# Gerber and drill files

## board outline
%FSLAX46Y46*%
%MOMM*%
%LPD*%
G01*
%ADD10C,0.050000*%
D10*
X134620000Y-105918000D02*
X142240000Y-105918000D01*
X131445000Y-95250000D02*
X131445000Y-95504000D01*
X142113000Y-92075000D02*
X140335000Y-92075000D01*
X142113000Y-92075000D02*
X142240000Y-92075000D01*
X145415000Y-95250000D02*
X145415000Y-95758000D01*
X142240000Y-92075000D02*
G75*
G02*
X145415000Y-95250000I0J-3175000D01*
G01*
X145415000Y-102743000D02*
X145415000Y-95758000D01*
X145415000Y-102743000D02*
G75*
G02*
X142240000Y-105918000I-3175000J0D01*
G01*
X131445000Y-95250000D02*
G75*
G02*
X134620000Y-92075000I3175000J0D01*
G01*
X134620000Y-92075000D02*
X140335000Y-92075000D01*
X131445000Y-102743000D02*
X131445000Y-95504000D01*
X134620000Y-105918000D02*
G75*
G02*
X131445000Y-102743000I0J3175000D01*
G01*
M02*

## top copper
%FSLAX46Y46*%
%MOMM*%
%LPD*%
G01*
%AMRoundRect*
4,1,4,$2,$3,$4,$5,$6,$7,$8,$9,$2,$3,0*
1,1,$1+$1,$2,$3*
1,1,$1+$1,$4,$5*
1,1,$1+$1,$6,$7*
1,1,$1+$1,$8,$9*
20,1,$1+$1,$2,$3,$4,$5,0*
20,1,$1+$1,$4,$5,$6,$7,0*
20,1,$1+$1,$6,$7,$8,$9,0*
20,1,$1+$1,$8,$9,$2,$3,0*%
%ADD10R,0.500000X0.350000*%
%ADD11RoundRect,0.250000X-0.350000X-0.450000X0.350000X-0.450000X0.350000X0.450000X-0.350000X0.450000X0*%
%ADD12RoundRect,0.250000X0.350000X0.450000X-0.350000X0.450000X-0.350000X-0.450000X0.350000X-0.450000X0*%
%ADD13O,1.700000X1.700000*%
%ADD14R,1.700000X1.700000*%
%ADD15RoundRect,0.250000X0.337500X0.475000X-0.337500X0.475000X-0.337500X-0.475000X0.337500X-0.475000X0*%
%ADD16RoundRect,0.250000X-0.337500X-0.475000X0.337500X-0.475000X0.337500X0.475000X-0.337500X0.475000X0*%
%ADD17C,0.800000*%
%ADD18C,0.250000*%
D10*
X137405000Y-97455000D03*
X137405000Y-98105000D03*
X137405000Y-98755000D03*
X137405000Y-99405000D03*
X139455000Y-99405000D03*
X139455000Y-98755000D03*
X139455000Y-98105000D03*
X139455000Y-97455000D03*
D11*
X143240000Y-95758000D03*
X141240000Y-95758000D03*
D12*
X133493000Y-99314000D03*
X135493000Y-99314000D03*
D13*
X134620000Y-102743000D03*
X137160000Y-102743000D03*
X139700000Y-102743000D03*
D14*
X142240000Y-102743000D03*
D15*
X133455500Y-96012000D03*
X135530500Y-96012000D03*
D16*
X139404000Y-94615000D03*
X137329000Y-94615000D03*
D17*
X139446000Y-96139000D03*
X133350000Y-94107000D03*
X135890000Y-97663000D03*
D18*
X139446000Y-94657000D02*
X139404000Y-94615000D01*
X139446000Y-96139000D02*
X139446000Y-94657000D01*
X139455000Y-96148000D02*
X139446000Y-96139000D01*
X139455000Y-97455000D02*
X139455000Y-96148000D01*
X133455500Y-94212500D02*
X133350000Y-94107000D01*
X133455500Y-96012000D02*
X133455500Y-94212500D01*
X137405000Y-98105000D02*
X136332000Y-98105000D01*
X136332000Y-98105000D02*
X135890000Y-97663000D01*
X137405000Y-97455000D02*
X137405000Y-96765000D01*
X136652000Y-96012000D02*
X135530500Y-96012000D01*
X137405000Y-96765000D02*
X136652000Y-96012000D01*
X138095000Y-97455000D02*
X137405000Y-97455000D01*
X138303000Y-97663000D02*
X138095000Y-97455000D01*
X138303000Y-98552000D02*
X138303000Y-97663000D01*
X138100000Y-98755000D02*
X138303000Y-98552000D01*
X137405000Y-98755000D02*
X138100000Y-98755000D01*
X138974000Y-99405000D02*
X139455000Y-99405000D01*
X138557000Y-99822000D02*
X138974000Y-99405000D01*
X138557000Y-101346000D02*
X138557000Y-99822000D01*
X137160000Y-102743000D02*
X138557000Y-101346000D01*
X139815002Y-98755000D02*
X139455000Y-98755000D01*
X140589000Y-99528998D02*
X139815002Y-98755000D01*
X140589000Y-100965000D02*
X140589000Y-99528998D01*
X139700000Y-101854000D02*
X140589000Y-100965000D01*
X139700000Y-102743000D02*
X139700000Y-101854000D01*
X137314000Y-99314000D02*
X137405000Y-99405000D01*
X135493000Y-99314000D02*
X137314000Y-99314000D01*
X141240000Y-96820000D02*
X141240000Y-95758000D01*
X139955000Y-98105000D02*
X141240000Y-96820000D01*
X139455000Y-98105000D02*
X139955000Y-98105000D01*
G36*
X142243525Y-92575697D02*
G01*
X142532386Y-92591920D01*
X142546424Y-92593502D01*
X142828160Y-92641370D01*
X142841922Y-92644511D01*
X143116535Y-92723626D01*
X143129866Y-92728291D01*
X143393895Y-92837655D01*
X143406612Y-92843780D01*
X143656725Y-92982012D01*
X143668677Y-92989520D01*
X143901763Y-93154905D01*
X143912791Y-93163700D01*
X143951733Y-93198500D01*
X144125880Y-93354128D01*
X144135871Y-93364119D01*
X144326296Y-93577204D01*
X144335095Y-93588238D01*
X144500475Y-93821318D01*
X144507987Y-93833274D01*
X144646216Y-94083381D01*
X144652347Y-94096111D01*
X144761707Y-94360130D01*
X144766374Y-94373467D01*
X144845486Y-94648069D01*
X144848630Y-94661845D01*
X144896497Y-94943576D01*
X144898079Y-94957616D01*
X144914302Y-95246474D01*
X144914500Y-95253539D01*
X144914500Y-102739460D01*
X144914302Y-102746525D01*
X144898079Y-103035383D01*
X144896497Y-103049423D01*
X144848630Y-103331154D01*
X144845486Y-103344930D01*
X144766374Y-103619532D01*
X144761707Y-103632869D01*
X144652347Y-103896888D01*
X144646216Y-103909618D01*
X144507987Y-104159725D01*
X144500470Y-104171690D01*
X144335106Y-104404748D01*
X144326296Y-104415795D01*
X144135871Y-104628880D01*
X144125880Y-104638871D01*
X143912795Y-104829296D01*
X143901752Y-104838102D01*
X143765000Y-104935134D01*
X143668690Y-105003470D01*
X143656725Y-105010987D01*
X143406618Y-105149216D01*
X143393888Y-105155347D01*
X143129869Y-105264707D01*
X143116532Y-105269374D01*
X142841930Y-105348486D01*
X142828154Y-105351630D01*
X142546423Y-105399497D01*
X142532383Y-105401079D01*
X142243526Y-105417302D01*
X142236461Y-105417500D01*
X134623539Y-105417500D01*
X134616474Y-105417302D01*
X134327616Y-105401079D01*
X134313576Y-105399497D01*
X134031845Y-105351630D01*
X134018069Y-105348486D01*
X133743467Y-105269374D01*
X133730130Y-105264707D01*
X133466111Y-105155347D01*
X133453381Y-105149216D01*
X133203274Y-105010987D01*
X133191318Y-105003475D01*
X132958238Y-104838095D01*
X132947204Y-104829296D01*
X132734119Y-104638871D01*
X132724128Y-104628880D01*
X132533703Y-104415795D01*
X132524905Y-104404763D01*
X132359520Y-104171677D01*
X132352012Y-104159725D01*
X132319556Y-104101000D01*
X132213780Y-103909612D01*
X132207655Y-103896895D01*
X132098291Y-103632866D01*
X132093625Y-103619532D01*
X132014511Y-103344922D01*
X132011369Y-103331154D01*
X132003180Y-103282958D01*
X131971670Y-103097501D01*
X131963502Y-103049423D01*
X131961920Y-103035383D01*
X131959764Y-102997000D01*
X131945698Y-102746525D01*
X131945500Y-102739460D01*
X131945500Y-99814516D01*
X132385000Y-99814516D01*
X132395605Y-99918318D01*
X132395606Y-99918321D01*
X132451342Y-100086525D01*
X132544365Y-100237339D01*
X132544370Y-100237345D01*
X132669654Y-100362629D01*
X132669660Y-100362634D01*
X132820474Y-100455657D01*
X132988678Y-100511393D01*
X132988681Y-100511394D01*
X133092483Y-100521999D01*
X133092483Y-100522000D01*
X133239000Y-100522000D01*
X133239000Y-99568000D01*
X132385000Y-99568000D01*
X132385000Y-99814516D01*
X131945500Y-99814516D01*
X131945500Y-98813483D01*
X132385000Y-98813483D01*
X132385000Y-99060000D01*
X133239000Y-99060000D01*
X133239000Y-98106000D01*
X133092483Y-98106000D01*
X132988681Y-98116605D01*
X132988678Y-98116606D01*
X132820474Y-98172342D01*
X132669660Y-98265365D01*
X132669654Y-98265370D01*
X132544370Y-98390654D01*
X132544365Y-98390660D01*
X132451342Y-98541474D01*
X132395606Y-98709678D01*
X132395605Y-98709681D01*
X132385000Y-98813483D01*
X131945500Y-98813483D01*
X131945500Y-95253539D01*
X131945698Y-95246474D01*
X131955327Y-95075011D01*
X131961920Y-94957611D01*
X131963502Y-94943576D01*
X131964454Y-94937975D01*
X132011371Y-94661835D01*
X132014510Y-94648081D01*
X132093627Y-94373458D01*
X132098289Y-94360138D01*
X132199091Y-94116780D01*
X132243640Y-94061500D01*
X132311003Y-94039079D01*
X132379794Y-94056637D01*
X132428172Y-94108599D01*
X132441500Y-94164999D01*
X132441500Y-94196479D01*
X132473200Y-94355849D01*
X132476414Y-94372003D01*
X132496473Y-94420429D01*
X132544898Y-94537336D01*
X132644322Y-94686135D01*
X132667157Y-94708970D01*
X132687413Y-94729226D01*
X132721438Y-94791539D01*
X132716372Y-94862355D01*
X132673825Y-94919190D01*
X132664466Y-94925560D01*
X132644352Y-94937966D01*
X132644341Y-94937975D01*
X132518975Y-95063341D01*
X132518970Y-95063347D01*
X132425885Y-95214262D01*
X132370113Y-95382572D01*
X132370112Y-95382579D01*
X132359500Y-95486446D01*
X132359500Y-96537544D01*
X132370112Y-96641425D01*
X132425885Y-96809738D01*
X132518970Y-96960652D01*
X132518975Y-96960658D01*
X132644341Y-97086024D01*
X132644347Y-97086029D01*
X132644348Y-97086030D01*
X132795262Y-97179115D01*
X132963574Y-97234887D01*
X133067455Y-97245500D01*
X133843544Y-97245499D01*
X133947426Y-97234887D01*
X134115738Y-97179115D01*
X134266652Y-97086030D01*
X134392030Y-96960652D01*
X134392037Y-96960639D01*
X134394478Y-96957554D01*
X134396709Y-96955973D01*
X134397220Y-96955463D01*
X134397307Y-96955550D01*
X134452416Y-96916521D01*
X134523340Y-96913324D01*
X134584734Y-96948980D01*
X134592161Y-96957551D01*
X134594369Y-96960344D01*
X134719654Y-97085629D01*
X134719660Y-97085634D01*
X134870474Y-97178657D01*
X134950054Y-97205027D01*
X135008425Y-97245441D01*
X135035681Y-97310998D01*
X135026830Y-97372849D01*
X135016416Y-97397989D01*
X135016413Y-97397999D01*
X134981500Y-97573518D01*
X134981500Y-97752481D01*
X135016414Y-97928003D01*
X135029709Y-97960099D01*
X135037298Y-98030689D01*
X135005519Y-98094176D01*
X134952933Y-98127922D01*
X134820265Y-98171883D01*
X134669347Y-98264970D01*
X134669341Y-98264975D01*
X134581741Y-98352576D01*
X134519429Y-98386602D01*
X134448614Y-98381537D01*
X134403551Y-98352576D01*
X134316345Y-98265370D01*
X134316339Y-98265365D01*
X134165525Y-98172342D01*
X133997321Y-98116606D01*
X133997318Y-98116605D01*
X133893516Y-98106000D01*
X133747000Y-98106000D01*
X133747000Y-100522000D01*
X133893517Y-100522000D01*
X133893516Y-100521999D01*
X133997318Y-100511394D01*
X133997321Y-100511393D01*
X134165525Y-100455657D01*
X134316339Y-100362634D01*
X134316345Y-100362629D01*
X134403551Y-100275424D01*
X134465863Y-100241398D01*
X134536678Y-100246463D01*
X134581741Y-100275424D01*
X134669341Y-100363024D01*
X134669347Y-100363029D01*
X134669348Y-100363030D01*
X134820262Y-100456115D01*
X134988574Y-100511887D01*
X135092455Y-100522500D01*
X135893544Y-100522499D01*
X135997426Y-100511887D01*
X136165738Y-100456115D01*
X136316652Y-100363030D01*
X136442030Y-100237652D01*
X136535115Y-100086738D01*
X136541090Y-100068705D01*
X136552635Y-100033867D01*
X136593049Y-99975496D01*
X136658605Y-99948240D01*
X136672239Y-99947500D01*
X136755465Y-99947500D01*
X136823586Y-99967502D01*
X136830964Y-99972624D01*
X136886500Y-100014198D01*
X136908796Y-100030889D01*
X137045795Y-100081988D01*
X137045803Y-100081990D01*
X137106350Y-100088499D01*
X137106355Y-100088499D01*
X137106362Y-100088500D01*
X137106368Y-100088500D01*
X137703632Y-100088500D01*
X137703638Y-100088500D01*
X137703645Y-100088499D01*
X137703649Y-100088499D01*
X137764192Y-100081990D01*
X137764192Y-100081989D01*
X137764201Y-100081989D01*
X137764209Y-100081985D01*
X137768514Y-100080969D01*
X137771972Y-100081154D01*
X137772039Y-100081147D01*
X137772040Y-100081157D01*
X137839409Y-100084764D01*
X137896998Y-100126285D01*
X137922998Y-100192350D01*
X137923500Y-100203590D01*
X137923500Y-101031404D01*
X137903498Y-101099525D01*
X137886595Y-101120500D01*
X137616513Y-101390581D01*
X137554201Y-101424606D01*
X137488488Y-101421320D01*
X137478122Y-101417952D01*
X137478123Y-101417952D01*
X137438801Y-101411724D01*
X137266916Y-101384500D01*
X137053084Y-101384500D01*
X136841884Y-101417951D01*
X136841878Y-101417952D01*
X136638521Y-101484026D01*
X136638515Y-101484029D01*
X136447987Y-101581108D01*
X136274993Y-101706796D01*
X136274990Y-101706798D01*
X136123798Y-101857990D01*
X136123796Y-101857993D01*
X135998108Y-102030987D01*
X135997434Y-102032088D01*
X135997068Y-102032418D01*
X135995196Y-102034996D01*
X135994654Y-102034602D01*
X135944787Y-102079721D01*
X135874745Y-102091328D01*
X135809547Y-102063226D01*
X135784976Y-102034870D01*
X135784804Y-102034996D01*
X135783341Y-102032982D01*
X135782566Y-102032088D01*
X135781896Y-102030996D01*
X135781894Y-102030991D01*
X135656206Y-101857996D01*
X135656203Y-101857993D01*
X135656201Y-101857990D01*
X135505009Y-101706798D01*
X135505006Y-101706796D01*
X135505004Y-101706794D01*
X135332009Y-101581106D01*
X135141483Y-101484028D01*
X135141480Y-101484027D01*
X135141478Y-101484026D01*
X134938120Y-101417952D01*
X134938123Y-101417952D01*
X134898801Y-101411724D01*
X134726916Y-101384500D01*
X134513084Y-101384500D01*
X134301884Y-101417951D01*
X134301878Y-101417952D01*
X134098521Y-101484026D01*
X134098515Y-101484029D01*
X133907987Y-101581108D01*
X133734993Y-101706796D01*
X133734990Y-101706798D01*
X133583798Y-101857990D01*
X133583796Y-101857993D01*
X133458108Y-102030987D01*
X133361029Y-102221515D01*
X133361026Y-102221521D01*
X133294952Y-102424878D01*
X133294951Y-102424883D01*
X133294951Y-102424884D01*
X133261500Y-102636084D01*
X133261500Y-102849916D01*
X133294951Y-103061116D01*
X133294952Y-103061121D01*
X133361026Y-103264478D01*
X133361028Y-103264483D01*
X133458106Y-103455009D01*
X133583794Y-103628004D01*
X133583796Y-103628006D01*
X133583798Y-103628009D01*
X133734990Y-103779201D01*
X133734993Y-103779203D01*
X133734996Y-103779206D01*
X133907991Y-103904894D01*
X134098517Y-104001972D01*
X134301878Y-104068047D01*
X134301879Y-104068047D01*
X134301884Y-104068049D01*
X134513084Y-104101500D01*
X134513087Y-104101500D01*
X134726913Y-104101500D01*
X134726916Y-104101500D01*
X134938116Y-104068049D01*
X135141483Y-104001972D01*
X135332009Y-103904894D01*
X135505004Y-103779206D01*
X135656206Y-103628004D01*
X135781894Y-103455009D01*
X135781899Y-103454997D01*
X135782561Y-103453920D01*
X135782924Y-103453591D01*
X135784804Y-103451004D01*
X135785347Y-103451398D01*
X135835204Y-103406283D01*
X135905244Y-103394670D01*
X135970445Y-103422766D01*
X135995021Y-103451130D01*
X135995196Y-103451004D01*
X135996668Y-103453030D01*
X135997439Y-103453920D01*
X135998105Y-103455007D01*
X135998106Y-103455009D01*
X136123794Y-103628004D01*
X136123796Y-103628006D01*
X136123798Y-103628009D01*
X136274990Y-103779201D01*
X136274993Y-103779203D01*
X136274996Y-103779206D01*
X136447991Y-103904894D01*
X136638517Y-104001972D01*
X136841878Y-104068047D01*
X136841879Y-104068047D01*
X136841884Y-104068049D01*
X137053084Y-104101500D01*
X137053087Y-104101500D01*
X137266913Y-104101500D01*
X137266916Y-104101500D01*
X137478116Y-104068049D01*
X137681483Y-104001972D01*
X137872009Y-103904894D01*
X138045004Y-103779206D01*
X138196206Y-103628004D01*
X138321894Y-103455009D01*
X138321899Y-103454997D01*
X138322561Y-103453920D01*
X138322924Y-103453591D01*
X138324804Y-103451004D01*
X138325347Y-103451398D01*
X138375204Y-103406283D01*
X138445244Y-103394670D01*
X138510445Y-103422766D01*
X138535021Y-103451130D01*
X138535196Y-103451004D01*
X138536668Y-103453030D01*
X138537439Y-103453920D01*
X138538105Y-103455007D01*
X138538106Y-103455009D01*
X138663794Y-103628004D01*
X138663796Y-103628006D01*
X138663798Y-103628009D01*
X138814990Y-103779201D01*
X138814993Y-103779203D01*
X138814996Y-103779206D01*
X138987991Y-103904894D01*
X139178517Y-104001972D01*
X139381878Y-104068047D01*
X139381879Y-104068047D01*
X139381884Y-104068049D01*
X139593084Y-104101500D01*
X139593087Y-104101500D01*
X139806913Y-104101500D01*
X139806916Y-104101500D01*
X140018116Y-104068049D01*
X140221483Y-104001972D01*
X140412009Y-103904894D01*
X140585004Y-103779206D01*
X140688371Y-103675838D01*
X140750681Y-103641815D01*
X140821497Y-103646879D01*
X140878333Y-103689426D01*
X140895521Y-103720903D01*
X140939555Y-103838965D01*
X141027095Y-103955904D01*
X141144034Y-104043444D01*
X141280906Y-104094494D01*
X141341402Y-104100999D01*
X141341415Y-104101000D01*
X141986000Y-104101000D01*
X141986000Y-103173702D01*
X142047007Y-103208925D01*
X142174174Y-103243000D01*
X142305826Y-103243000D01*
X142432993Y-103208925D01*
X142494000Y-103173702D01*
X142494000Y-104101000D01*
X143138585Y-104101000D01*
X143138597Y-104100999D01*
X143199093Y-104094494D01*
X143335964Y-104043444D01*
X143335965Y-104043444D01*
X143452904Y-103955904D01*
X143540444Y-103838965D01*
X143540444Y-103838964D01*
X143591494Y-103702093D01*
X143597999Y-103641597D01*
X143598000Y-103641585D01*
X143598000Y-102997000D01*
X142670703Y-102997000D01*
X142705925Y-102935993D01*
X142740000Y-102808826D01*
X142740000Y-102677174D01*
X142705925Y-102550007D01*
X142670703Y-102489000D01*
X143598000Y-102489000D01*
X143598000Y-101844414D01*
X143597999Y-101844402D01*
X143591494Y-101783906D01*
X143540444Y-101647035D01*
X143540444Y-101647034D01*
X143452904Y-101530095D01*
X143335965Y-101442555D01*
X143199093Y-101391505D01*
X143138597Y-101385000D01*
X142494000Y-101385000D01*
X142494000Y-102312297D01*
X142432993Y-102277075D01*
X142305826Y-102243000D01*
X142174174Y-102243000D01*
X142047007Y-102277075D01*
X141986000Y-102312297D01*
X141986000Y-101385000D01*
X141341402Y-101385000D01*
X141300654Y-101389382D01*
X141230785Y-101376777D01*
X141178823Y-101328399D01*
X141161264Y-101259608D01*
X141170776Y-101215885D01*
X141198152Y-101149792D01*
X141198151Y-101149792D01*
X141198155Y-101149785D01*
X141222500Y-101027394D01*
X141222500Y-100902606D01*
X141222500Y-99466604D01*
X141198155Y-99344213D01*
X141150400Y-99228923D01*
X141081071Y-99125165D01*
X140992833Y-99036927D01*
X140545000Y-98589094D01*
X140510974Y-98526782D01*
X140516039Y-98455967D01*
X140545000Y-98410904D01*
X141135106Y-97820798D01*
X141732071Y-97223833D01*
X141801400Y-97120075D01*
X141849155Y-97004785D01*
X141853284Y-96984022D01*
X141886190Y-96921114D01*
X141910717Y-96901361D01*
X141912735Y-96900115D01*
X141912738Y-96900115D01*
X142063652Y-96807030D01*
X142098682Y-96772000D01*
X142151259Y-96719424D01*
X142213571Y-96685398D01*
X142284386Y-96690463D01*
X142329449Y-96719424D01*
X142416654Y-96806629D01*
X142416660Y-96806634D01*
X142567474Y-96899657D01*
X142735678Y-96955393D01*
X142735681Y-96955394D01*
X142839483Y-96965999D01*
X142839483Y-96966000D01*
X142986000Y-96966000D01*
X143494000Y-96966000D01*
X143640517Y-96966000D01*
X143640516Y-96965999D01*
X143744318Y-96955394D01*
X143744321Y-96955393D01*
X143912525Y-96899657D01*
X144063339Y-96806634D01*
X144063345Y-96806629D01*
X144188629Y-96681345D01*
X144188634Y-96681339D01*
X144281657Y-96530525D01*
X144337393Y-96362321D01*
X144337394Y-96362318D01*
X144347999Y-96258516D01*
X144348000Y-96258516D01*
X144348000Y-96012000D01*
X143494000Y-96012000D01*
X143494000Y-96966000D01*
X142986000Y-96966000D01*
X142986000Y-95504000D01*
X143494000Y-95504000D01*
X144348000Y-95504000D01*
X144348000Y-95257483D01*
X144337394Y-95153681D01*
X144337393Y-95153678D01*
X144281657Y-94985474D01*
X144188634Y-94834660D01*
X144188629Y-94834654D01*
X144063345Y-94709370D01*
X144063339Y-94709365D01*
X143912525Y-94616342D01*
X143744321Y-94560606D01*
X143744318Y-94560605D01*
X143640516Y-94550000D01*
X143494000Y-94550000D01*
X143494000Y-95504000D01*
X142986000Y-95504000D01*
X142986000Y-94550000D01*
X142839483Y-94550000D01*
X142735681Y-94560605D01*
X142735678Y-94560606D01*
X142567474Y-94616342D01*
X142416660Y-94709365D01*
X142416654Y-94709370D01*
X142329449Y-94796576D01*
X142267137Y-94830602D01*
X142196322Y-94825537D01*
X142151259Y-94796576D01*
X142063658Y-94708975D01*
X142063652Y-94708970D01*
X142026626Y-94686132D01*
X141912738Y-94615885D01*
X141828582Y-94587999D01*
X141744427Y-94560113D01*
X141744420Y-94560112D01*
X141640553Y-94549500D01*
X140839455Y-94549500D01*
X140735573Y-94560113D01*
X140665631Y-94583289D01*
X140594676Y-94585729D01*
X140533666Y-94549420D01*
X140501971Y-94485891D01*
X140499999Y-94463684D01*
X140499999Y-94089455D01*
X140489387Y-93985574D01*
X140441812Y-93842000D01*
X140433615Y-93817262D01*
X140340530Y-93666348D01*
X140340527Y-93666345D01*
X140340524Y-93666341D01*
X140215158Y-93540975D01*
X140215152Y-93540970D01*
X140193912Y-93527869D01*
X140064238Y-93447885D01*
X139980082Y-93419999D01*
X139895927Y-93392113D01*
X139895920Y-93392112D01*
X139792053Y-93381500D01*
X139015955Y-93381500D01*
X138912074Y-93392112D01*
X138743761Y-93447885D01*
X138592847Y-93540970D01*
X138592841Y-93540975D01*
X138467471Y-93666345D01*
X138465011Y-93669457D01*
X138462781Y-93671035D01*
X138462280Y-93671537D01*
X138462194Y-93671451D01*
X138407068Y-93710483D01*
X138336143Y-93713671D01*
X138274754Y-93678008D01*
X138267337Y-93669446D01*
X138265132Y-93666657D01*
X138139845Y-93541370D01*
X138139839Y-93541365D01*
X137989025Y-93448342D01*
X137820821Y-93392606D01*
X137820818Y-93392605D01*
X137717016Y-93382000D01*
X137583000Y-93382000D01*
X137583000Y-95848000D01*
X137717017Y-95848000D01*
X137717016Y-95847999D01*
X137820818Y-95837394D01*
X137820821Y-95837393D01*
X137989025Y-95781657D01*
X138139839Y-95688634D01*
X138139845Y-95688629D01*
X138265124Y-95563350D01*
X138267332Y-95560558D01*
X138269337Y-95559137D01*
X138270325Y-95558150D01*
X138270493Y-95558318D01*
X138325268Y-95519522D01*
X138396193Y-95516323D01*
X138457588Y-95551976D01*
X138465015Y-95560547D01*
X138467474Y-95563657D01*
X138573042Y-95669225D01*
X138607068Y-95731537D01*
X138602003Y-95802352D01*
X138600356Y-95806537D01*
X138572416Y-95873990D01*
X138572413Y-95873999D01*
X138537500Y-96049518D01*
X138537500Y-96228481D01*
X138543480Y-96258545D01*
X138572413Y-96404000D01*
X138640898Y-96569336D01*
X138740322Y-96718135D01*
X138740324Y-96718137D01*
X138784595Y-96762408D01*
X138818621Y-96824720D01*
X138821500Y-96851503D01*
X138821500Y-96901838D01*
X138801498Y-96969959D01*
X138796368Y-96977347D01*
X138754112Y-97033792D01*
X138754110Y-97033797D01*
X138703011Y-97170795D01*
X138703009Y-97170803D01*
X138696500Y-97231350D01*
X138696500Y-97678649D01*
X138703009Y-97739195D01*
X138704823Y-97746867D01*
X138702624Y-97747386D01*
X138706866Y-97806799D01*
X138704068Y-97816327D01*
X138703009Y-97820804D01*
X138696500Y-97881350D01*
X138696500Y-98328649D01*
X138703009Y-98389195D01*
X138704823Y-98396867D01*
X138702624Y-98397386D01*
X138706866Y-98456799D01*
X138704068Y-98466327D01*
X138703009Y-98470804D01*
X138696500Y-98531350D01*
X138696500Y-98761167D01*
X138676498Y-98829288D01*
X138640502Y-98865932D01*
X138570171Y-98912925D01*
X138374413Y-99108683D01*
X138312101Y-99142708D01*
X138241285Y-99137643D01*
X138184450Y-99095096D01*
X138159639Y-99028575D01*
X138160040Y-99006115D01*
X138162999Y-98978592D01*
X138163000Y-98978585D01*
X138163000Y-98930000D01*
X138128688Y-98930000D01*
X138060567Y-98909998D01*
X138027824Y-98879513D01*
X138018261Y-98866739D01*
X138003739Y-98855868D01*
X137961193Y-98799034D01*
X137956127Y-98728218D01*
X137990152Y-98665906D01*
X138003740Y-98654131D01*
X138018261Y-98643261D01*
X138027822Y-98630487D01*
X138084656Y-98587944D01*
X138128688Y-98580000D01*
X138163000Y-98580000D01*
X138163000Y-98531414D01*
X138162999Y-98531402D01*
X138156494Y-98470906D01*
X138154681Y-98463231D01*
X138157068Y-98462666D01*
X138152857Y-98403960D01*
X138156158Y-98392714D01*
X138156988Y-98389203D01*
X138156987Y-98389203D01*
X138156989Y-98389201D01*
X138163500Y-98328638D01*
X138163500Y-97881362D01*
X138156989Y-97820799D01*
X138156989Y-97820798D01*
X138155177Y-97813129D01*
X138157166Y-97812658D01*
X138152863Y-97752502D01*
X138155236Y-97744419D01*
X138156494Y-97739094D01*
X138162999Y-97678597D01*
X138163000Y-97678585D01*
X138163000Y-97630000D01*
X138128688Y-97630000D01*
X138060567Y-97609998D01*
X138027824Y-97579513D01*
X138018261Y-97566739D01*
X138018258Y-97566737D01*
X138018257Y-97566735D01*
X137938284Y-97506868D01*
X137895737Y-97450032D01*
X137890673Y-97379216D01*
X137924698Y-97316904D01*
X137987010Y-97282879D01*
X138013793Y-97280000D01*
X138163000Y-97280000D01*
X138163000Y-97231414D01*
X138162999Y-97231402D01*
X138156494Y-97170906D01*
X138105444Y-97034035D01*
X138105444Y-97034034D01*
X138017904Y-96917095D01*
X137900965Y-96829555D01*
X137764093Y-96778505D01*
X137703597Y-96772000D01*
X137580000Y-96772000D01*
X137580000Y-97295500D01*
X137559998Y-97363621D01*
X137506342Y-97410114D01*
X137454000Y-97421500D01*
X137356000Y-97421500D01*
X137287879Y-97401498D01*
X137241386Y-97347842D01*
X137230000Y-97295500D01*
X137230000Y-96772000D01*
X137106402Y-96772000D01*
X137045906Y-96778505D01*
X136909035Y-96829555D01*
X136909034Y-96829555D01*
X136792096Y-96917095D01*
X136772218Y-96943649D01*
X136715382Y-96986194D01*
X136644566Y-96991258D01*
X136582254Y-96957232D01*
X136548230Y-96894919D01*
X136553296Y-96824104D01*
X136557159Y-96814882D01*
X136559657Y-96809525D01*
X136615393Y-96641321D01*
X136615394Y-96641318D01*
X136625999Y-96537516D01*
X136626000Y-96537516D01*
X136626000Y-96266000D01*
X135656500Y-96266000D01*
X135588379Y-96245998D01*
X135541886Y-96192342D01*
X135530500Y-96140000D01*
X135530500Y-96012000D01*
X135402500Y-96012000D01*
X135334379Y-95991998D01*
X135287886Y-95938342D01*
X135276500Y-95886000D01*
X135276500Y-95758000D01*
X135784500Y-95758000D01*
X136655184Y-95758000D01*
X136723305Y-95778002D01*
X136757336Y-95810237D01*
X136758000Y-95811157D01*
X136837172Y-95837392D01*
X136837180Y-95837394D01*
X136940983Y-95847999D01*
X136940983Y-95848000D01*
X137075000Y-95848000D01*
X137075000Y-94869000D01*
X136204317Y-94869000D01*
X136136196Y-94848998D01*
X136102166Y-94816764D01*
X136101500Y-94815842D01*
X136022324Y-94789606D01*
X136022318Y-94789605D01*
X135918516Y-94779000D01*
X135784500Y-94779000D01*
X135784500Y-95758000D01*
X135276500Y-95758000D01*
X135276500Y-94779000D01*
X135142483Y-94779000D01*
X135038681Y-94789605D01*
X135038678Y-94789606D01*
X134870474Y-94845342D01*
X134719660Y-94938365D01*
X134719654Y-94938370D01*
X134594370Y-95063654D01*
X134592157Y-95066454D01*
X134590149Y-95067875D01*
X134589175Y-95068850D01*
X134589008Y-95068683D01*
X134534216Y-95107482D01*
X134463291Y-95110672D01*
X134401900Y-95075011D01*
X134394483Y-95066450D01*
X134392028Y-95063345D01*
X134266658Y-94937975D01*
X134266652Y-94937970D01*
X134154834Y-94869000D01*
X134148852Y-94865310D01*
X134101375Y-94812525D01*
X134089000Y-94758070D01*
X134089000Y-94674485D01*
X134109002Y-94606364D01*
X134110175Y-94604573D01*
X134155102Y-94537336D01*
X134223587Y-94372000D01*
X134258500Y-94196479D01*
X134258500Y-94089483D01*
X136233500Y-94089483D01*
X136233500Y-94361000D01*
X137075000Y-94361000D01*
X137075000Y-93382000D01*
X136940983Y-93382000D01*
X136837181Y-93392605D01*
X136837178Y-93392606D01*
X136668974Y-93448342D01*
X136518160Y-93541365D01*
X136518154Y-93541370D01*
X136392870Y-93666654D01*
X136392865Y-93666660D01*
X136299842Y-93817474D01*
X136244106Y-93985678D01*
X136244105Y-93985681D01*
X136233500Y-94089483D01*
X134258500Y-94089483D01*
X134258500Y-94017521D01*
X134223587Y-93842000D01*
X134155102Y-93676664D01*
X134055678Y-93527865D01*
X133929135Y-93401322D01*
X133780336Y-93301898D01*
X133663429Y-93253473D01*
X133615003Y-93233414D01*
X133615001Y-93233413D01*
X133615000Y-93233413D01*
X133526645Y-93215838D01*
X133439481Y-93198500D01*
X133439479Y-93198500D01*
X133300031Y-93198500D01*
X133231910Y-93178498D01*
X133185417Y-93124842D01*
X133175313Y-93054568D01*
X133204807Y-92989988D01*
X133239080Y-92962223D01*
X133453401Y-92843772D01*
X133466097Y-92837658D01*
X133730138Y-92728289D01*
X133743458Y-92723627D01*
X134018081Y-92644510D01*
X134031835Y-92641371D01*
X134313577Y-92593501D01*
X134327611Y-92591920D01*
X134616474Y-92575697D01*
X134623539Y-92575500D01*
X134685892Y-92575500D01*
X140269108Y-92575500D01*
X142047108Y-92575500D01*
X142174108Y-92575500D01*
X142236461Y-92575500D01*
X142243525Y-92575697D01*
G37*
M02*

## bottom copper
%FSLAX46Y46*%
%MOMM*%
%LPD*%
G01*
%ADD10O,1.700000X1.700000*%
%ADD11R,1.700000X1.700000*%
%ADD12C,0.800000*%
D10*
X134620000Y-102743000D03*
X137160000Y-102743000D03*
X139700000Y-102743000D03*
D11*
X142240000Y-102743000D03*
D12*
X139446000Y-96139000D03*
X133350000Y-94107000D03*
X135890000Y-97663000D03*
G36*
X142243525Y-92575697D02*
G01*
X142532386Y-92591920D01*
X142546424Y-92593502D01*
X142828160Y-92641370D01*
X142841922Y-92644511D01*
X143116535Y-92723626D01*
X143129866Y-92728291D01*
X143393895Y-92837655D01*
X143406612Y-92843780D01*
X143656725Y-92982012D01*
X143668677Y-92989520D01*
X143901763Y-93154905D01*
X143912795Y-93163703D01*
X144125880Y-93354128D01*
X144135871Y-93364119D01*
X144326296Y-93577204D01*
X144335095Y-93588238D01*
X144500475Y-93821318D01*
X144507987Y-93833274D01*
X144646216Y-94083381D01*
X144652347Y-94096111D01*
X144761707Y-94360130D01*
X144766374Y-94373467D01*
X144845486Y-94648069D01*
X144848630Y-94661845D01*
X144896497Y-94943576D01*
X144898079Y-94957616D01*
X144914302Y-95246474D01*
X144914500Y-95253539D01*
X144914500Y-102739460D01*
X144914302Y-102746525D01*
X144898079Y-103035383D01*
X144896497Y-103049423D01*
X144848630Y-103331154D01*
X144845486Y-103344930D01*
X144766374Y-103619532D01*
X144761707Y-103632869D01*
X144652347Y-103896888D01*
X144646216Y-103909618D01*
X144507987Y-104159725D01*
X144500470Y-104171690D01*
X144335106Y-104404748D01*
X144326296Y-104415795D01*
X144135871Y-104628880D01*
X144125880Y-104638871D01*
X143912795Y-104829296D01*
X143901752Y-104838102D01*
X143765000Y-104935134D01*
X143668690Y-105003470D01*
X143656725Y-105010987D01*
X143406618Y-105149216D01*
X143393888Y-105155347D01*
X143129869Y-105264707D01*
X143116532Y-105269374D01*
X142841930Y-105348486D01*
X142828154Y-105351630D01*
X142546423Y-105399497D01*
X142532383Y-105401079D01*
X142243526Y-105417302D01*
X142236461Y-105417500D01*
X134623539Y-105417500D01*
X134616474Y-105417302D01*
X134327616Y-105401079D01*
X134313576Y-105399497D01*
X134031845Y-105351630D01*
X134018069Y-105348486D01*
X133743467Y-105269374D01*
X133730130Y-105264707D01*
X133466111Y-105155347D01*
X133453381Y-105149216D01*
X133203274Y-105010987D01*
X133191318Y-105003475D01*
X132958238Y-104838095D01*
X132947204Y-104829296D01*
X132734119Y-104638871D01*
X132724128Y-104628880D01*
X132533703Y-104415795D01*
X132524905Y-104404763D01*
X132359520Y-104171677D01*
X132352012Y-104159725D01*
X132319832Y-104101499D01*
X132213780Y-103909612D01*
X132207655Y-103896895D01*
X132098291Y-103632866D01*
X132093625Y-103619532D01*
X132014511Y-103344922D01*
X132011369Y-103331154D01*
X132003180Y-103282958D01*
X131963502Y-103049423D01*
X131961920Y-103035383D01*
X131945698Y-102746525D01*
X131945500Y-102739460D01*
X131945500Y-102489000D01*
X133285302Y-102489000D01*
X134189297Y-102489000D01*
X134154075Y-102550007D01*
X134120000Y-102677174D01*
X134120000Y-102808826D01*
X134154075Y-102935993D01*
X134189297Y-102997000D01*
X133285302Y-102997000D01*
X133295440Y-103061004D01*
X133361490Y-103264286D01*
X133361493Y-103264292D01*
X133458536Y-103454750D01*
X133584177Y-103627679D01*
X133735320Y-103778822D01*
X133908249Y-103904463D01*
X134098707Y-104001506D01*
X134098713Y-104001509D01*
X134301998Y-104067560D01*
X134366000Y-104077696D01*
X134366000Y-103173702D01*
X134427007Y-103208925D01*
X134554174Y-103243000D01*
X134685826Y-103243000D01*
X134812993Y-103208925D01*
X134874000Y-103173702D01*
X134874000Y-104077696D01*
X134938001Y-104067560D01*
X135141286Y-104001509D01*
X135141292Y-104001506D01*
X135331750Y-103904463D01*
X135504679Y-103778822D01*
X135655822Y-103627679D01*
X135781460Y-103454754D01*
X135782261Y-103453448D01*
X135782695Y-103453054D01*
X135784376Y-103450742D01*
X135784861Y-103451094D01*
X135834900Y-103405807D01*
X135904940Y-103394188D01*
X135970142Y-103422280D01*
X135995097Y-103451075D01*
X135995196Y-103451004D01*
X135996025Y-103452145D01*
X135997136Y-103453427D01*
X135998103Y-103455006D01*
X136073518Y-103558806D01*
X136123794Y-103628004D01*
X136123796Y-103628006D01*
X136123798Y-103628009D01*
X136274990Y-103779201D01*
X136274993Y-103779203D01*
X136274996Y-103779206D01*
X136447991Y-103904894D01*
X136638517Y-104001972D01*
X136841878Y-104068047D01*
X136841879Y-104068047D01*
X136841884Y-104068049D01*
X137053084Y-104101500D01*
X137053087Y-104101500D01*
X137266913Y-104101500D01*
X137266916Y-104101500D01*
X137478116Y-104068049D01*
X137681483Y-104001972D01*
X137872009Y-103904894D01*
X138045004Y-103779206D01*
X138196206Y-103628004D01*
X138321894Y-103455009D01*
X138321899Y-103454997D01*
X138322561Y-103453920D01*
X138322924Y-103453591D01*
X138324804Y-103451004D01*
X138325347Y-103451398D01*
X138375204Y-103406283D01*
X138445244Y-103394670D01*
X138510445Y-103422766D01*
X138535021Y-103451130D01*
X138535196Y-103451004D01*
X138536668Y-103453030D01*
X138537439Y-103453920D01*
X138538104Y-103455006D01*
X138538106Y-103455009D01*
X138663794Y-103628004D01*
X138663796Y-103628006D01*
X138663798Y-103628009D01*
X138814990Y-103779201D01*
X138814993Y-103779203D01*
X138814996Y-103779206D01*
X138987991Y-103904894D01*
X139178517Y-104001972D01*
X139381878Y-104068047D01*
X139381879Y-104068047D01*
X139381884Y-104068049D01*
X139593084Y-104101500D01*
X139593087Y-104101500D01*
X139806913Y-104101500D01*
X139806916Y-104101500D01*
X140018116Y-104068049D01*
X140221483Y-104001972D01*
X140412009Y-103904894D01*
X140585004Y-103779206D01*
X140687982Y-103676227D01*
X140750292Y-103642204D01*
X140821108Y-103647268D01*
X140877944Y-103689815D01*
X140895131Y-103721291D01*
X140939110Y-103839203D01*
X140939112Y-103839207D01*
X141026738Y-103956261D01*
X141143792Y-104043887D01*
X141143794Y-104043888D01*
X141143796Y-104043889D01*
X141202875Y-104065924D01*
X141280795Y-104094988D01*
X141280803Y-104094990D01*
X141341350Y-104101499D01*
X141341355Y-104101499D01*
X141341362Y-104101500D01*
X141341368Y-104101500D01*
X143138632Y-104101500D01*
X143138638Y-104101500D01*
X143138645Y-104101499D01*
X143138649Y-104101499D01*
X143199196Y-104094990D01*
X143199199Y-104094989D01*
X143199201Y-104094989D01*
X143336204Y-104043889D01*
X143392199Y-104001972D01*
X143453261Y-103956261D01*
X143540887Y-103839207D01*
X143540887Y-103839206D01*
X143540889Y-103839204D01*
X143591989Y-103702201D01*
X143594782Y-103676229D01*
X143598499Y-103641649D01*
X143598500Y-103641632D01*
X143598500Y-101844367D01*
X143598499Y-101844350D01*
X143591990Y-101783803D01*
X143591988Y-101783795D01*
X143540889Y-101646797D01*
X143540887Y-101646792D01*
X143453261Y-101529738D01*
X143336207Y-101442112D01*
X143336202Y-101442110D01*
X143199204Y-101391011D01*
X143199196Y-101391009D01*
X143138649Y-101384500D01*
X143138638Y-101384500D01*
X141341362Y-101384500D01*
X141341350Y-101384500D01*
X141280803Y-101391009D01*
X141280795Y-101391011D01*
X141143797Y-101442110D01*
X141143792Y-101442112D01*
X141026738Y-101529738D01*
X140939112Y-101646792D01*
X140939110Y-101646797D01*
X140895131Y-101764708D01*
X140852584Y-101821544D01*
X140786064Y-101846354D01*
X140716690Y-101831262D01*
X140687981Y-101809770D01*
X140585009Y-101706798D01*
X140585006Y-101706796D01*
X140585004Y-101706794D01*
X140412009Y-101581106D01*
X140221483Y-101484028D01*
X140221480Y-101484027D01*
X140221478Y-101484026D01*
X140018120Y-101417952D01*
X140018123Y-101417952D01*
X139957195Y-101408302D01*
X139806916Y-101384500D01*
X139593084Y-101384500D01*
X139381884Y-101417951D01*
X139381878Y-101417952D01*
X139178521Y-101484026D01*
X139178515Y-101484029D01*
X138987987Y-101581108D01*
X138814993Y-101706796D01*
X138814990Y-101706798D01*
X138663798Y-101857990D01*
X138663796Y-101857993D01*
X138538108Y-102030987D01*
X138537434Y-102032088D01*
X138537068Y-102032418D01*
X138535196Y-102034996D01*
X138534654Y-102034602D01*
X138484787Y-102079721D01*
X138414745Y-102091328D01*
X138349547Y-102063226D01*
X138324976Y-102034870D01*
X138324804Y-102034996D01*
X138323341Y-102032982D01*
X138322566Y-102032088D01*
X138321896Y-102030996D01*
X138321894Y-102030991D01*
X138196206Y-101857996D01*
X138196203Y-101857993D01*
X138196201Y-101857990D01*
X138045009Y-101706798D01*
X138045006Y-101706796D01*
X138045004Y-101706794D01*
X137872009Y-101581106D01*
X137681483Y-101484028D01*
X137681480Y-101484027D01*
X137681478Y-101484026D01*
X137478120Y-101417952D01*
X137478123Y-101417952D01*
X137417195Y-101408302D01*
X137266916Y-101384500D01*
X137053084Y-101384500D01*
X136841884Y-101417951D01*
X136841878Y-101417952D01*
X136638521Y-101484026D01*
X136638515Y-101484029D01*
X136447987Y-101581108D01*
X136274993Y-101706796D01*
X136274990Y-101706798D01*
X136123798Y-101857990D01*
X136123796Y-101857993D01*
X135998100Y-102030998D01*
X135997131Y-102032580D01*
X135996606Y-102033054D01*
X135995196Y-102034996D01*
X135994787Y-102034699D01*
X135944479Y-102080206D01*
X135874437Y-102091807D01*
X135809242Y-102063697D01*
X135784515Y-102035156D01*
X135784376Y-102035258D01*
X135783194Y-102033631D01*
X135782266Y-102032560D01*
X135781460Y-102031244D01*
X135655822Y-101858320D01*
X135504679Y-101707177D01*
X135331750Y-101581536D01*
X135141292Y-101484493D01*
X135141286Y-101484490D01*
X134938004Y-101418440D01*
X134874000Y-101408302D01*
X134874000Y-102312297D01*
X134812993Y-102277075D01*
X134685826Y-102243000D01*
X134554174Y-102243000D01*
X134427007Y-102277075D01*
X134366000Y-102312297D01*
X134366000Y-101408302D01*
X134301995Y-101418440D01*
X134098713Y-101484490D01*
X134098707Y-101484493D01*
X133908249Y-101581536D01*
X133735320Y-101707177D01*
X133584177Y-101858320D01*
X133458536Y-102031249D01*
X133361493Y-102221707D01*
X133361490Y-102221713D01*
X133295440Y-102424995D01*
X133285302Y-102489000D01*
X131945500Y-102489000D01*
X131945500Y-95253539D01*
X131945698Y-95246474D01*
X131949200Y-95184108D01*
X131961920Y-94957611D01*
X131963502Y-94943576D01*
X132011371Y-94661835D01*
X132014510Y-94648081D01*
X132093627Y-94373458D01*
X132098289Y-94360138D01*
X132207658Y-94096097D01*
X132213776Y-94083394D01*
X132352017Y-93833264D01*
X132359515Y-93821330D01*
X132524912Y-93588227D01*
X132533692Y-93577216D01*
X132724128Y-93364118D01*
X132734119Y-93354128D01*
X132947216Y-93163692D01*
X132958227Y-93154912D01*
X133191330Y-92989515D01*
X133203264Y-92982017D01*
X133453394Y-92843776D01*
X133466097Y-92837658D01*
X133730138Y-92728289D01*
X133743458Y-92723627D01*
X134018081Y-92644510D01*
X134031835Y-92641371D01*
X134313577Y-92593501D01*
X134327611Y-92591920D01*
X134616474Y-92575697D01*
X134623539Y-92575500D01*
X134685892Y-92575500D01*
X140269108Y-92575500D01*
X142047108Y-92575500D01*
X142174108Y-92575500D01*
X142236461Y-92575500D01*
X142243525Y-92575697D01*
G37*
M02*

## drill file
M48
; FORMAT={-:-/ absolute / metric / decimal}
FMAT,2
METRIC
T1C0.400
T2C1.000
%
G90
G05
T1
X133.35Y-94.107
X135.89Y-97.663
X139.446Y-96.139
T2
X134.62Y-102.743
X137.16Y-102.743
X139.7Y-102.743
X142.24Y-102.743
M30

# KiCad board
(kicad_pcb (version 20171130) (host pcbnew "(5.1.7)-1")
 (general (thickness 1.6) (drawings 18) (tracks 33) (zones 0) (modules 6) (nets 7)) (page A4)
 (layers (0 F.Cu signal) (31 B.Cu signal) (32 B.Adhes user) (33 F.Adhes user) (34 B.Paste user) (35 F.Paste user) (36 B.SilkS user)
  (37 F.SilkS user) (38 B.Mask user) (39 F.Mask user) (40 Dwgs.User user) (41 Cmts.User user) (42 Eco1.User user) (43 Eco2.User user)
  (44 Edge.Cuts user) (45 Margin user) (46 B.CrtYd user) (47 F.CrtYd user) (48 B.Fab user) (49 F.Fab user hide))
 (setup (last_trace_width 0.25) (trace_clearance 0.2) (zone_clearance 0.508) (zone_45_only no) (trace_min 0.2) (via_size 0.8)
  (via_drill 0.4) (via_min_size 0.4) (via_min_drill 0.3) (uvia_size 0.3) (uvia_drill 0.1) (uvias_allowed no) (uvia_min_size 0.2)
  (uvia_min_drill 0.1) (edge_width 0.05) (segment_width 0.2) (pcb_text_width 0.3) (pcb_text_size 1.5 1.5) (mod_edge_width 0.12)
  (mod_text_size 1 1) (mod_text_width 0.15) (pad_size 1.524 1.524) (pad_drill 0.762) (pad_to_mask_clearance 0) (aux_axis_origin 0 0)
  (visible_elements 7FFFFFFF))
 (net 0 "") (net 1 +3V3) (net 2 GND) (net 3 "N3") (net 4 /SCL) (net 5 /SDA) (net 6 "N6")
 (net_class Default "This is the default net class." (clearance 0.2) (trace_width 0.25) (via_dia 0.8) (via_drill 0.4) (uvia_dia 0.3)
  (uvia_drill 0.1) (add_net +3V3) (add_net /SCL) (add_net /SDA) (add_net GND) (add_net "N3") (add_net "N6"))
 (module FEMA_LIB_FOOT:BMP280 (layer F.Cu) (at 138.43 98.425)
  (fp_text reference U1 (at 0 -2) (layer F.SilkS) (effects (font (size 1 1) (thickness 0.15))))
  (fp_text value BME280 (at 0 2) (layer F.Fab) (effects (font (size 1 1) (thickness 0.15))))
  (pad 8 smd rect (at -1.025 -0.97) (size 0.5 0.35) (layers F.Cu F.Paste F.Mask) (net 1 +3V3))
  (pad 7 smd rect (at -1.025 -0.32) (size 0.5 0.35) (layers F.Cu F.Paste F.Mask) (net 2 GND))
  (pad 6 smd rect (at -1.025 0.33) (size 0.5 0.35) (layers F.Cu F.Paste F.Mask) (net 1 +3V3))
  (pad 5 smd rect (at -1.025 0.98) (size 0.5 0.35) (layers F.Cu F.Paste F.Mask) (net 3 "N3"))
  (pad 4 smd rect (at 1.025 0.98) (size 0.5 0.35) (layers F.Cu F.Paste F.Mask) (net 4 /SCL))
  (pad 3 smd rect (at 1.025 0.33) (size 0.5 0.35) (layers F.Cu F.Paste F.Mask) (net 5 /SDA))
  (pad 2 smd rect (at 1.025 -0.32) (size 0.5 0.35) (layers F.Cu F.Paste F.Mask) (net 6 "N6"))
  (pad 1 smd rect (at 1.025 -0.97) (size 0.5 0.35) (layers F.Cu F.Paste F.Mask) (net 2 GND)))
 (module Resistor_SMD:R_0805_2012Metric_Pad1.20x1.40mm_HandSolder (layer F.Cu) (at 142.24 95.758)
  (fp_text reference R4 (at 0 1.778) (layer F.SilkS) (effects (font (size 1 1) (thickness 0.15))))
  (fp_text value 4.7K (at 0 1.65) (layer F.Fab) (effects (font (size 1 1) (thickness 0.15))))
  (pad 2 smd roundrect (at 1 0) (size 1.2 1.4) (layers F.Cu F.Paste F.Mask) (roundrect_rratio 0.208333) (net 1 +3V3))
  (pad 1 smd roundrect (at -1 0) (size 1.2 1.4) (layers F.Cu F.Paste F.Mask) (roundrect_rratio 0.208333) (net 6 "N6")))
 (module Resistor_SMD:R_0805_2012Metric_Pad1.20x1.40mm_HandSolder (layer F.Cu) (at 134.493 99.314 180)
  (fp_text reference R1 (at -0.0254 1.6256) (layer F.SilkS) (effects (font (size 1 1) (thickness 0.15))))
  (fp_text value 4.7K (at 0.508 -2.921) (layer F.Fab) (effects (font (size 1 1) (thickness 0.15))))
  (pad 2 smd roundrect (at 1 0 180) (size 1.2 1.4) (layers F.Cu F.Paste F.Mask) (roundrect_rratio 0.208333) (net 1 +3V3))
  (pad 1 smd roundrect (at -1 0 180) (size 1.2 1.4) (layers F.Cu F.Paste F.Mask) (roundrect_rratio 0.208333) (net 3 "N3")))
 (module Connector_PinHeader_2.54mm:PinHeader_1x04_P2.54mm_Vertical (layer F.Cu) (at 142.24 102.743 270)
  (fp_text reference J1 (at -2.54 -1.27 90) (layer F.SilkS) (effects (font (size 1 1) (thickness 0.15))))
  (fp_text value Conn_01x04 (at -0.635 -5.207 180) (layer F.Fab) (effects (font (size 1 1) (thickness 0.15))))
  (pad 4 thru_hole oval (at 0 7.62 270) (size 1.7 1.7) (drill 1) (layers *.Cu *.Mask) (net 2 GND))
  (pad 3 thru_hole oval (at 0 5.08 270) (size 1.7 1.7) (drill 1) (layers *.Cu *.Mask) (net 4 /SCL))
  (pad 2 thru_hole oval (at 0 2.54 270) (size 1.7 1.7) (drill 1) (layers *.Cu *.Mask) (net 5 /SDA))
  (pad 1 thru_hole rect (at 0 0 270) (size 1.7 1.7) (drill 1) (layers *.Cu *.Mask) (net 1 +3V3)))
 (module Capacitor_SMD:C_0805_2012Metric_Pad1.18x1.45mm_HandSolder (layer F.Cu) (at 134.493 96.012 180)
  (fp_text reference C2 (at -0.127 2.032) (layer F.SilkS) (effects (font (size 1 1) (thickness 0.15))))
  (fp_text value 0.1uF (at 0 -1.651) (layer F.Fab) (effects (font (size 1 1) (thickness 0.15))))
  (pad 2 smd roundrect (at 1.0375 0 180) (size 1.175 1.45) (layers F.Cu F.Paste F.Mask) (roundrect_rratio 0.212766) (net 2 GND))
  (pad 1 smd roundrect (at -1.0375 0 180) (size 1.175 1.45) (layers F.Cu F.Paste F.Mask) (roundrect_rratio 0.212766) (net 1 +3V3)))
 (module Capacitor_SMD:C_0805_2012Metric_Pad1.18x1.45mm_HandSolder (layer F.Cu) (at 138.3665 94.615)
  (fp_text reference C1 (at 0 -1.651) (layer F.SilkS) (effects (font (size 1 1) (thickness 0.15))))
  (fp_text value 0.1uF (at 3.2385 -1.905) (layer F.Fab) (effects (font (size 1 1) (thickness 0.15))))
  (pad 2 smd roundrect (at 1.0375 0) (size 1.175 1.45) (layers F.Cu F.Paste F.Mask) (roundrect_rratio 0.212766) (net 2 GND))
  (pad 1 smd roundrect (at -1.0375 0) (size 1.175 1.45) (layers F.Cu F.Paste F.Mask) (roundrect_rratio 0.212766) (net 1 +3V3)))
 (gr_line (start 134.62 105.918) (end 142.24 105.918) (layer Edge.Cuts) (width 0.05))
 (gr_line (start 131.445 95.25) (end 131.445 95.504) (layer Edge.Cuts) (width 0.05))
 (gr_line (start 142.113 92.075) (end 140.335 92.075) (layer Edge.Cuts) (width 0.05))
 (gr_line (start 142.113 92.075) (end 142.24 92.075) (layer Edge.Cuts) (width 0.05))
 (gr_line (start 145.415 95.25) (end 145.415 95.758) (layer Edge.Cuts) (width 0.05))
 (gr_arc (start 142.24 95.25) (end 145.415 95.25) (angle -90) (layer Edge.Cuts) (width 0.05))
 (gr_line (start 145.415 102.743) (end 145.415 95.758) (layer Edge.Cuts) (width 0.05))
 (gr_arc (start 142.24 102.743) (end 142.24 105.918) (angle -90) (layer Edge.Cuts) (width 0.05))
 (gr_arc (start 134.62 95.25) (end 134.62 92.075) (angle -90) (layer Edge.Cuts) (width 0.05))
 (gr_line (start 134.62 92.075) (end 140.335 92.075) (layer Edge.Cuts) (width 0.05))
 (gr_line (start 131.445 102.743) (end 131.445 95.504) (layer Edge.Cuts) (width 0.05))
 (gr_arc (start 134.62 102.743) (end 131.445 102.743) (angle -90) (layer Edge.Cuts) (width 0.05))
 (via (at 139.446 96.139) (size 0.8) (drill 0.4) (layers F.Cu B.Cu) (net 2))
 (segment (start 139.446 94.657) (end 139.404 94.615) (width 0.25) (layer F.Cu) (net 2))
 (segment (start 139.446 96.139) (end 139.446 94.657) (width 0.25) (layer F.Cu) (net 2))
 (segment (start 139.455 96.148) (end 139.446 96.139) (width 0.25) (layer F.Cu) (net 2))
 (segment (start 139.455 97.455) (end 139.455 96.148) (width 0.25) (layer F.Cu) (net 2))
 (via (at 133.35 94.107) (size 0.8) (drill 0.4) (layers F.Cu B.Cu) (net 2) (status 1000000))
 (segment (start 133.4555 94.2125) (end 133.35 94.107) (width 0.25) (layer F.Cu) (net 2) (status 1000000))
 (segment (start 133.4555 96.012) (end 133.4555 94.2125) (width 0.25) (layer F.Cu) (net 2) (status 1000000))
 (via (at 135.89 97.663) (size 0.8) (drill 0.4) (layers F.Cu B.Cu) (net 2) (status 1000000))
 (segment (start 137.405 98.105) (end 136.332 98.105) (width 0.25) (layer F.Cu) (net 2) (status 1000000))
 (segment (start 136.332 98.105) (end 135.89 97.663) (width 0.25) (layer F.Cu) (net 2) (status 1000000))
 (segment (start 137.405 97.455) (end 137.405 96.765) (width 0.25) (layer F.Cu) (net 1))
 (segment (start 136.652 96.012) (end 135.5305 96.012) (width 0.25) (layer F.Cu) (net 1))
 (segment (start 137.405 96.765) (end 136.652 96.012) (width 0.25) (layer F.Cu) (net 1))
 (segment (start 138.095 97.455) (end 137.405 97.455) (width 0.25) (layer F.Cu) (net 1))
 (segment (start 138.303 97.663) (end 138.095 97.455) (width 0.25) (layer F.Cu) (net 1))
 (segment (start 138.303 98.552) (end 138.303 97.663) (width 0.25) (layer F.Cu) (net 1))
 (segment (start 138.1 98.755) (end 138.303 98.552) (width 0.25) (layer F.Cu) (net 1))
 (segment (start 137.405 98.755) (end 138.1 98.755) (width 0.25) (layer F.Cu) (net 1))
 (segment (start 138.974 99.405) (end 139.455 99.405) (width 0.25) (layer F.Cu) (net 4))
 (segment (start 138.557 99.822) (end 138.974 99.405) (width 0.25) (layer F.Cu) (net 4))
 (segment (start 138.557 101.346) (end 138.557 99.822) (width 0.25) (layer F.Cu) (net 4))
 (segment (start 137.16 102.743) (end 138.557 101.346) (width 0.25) (layer F.Cu) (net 4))
 (segment (start 139.815002 98.755) (end 139.455 98.755) (width 0.25) (layer F.Cu) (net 5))
 (segment (start 140.589 99.528998) (end 139.815002 98.755) (width 0.25) (layer F.Cu) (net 5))
 (segment (start 140.589 100.965) (end 140.589 99.528998) (width 0.25) (layer F.Cu) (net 5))
 (segment (start 139.7 101.854) (end 140.589 100.965) (width 0.25) (layer F.Cu) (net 5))
 (segment (start 139.7 102.743) (end 139.7 101.854) (width 0.25) (layer F.Cu) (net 5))
 (segment (start 137.314 99.314) (end 137.405 99.405) (width 0.25) (layer F.Cu) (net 3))
 (segment (start 135.493 99.314) (end 137.314 99.314) (width 0.25) (layer F.Cu) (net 3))
 (segment (start 141.24 96.82) (end 141.24 95.758) (width 0.25) (layer F.Cu) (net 6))
 (segment (start 139.955 98.105) (end 141.24 96.82) (width 0.25) (layer F.Cu) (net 6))
 (segment (start 139.455 98.105) (end 139.955 98.105) (width 0.25) (layer F.Cu) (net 6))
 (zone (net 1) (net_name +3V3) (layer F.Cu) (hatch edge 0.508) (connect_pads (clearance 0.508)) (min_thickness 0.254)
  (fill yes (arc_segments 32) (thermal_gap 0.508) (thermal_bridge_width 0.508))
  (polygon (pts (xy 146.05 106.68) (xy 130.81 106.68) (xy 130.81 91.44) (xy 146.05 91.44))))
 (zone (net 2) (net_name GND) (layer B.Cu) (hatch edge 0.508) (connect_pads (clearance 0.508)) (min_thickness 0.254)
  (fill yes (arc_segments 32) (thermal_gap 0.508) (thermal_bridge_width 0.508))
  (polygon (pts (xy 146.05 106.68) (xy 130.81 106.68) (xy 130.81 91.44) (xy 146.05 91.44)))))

